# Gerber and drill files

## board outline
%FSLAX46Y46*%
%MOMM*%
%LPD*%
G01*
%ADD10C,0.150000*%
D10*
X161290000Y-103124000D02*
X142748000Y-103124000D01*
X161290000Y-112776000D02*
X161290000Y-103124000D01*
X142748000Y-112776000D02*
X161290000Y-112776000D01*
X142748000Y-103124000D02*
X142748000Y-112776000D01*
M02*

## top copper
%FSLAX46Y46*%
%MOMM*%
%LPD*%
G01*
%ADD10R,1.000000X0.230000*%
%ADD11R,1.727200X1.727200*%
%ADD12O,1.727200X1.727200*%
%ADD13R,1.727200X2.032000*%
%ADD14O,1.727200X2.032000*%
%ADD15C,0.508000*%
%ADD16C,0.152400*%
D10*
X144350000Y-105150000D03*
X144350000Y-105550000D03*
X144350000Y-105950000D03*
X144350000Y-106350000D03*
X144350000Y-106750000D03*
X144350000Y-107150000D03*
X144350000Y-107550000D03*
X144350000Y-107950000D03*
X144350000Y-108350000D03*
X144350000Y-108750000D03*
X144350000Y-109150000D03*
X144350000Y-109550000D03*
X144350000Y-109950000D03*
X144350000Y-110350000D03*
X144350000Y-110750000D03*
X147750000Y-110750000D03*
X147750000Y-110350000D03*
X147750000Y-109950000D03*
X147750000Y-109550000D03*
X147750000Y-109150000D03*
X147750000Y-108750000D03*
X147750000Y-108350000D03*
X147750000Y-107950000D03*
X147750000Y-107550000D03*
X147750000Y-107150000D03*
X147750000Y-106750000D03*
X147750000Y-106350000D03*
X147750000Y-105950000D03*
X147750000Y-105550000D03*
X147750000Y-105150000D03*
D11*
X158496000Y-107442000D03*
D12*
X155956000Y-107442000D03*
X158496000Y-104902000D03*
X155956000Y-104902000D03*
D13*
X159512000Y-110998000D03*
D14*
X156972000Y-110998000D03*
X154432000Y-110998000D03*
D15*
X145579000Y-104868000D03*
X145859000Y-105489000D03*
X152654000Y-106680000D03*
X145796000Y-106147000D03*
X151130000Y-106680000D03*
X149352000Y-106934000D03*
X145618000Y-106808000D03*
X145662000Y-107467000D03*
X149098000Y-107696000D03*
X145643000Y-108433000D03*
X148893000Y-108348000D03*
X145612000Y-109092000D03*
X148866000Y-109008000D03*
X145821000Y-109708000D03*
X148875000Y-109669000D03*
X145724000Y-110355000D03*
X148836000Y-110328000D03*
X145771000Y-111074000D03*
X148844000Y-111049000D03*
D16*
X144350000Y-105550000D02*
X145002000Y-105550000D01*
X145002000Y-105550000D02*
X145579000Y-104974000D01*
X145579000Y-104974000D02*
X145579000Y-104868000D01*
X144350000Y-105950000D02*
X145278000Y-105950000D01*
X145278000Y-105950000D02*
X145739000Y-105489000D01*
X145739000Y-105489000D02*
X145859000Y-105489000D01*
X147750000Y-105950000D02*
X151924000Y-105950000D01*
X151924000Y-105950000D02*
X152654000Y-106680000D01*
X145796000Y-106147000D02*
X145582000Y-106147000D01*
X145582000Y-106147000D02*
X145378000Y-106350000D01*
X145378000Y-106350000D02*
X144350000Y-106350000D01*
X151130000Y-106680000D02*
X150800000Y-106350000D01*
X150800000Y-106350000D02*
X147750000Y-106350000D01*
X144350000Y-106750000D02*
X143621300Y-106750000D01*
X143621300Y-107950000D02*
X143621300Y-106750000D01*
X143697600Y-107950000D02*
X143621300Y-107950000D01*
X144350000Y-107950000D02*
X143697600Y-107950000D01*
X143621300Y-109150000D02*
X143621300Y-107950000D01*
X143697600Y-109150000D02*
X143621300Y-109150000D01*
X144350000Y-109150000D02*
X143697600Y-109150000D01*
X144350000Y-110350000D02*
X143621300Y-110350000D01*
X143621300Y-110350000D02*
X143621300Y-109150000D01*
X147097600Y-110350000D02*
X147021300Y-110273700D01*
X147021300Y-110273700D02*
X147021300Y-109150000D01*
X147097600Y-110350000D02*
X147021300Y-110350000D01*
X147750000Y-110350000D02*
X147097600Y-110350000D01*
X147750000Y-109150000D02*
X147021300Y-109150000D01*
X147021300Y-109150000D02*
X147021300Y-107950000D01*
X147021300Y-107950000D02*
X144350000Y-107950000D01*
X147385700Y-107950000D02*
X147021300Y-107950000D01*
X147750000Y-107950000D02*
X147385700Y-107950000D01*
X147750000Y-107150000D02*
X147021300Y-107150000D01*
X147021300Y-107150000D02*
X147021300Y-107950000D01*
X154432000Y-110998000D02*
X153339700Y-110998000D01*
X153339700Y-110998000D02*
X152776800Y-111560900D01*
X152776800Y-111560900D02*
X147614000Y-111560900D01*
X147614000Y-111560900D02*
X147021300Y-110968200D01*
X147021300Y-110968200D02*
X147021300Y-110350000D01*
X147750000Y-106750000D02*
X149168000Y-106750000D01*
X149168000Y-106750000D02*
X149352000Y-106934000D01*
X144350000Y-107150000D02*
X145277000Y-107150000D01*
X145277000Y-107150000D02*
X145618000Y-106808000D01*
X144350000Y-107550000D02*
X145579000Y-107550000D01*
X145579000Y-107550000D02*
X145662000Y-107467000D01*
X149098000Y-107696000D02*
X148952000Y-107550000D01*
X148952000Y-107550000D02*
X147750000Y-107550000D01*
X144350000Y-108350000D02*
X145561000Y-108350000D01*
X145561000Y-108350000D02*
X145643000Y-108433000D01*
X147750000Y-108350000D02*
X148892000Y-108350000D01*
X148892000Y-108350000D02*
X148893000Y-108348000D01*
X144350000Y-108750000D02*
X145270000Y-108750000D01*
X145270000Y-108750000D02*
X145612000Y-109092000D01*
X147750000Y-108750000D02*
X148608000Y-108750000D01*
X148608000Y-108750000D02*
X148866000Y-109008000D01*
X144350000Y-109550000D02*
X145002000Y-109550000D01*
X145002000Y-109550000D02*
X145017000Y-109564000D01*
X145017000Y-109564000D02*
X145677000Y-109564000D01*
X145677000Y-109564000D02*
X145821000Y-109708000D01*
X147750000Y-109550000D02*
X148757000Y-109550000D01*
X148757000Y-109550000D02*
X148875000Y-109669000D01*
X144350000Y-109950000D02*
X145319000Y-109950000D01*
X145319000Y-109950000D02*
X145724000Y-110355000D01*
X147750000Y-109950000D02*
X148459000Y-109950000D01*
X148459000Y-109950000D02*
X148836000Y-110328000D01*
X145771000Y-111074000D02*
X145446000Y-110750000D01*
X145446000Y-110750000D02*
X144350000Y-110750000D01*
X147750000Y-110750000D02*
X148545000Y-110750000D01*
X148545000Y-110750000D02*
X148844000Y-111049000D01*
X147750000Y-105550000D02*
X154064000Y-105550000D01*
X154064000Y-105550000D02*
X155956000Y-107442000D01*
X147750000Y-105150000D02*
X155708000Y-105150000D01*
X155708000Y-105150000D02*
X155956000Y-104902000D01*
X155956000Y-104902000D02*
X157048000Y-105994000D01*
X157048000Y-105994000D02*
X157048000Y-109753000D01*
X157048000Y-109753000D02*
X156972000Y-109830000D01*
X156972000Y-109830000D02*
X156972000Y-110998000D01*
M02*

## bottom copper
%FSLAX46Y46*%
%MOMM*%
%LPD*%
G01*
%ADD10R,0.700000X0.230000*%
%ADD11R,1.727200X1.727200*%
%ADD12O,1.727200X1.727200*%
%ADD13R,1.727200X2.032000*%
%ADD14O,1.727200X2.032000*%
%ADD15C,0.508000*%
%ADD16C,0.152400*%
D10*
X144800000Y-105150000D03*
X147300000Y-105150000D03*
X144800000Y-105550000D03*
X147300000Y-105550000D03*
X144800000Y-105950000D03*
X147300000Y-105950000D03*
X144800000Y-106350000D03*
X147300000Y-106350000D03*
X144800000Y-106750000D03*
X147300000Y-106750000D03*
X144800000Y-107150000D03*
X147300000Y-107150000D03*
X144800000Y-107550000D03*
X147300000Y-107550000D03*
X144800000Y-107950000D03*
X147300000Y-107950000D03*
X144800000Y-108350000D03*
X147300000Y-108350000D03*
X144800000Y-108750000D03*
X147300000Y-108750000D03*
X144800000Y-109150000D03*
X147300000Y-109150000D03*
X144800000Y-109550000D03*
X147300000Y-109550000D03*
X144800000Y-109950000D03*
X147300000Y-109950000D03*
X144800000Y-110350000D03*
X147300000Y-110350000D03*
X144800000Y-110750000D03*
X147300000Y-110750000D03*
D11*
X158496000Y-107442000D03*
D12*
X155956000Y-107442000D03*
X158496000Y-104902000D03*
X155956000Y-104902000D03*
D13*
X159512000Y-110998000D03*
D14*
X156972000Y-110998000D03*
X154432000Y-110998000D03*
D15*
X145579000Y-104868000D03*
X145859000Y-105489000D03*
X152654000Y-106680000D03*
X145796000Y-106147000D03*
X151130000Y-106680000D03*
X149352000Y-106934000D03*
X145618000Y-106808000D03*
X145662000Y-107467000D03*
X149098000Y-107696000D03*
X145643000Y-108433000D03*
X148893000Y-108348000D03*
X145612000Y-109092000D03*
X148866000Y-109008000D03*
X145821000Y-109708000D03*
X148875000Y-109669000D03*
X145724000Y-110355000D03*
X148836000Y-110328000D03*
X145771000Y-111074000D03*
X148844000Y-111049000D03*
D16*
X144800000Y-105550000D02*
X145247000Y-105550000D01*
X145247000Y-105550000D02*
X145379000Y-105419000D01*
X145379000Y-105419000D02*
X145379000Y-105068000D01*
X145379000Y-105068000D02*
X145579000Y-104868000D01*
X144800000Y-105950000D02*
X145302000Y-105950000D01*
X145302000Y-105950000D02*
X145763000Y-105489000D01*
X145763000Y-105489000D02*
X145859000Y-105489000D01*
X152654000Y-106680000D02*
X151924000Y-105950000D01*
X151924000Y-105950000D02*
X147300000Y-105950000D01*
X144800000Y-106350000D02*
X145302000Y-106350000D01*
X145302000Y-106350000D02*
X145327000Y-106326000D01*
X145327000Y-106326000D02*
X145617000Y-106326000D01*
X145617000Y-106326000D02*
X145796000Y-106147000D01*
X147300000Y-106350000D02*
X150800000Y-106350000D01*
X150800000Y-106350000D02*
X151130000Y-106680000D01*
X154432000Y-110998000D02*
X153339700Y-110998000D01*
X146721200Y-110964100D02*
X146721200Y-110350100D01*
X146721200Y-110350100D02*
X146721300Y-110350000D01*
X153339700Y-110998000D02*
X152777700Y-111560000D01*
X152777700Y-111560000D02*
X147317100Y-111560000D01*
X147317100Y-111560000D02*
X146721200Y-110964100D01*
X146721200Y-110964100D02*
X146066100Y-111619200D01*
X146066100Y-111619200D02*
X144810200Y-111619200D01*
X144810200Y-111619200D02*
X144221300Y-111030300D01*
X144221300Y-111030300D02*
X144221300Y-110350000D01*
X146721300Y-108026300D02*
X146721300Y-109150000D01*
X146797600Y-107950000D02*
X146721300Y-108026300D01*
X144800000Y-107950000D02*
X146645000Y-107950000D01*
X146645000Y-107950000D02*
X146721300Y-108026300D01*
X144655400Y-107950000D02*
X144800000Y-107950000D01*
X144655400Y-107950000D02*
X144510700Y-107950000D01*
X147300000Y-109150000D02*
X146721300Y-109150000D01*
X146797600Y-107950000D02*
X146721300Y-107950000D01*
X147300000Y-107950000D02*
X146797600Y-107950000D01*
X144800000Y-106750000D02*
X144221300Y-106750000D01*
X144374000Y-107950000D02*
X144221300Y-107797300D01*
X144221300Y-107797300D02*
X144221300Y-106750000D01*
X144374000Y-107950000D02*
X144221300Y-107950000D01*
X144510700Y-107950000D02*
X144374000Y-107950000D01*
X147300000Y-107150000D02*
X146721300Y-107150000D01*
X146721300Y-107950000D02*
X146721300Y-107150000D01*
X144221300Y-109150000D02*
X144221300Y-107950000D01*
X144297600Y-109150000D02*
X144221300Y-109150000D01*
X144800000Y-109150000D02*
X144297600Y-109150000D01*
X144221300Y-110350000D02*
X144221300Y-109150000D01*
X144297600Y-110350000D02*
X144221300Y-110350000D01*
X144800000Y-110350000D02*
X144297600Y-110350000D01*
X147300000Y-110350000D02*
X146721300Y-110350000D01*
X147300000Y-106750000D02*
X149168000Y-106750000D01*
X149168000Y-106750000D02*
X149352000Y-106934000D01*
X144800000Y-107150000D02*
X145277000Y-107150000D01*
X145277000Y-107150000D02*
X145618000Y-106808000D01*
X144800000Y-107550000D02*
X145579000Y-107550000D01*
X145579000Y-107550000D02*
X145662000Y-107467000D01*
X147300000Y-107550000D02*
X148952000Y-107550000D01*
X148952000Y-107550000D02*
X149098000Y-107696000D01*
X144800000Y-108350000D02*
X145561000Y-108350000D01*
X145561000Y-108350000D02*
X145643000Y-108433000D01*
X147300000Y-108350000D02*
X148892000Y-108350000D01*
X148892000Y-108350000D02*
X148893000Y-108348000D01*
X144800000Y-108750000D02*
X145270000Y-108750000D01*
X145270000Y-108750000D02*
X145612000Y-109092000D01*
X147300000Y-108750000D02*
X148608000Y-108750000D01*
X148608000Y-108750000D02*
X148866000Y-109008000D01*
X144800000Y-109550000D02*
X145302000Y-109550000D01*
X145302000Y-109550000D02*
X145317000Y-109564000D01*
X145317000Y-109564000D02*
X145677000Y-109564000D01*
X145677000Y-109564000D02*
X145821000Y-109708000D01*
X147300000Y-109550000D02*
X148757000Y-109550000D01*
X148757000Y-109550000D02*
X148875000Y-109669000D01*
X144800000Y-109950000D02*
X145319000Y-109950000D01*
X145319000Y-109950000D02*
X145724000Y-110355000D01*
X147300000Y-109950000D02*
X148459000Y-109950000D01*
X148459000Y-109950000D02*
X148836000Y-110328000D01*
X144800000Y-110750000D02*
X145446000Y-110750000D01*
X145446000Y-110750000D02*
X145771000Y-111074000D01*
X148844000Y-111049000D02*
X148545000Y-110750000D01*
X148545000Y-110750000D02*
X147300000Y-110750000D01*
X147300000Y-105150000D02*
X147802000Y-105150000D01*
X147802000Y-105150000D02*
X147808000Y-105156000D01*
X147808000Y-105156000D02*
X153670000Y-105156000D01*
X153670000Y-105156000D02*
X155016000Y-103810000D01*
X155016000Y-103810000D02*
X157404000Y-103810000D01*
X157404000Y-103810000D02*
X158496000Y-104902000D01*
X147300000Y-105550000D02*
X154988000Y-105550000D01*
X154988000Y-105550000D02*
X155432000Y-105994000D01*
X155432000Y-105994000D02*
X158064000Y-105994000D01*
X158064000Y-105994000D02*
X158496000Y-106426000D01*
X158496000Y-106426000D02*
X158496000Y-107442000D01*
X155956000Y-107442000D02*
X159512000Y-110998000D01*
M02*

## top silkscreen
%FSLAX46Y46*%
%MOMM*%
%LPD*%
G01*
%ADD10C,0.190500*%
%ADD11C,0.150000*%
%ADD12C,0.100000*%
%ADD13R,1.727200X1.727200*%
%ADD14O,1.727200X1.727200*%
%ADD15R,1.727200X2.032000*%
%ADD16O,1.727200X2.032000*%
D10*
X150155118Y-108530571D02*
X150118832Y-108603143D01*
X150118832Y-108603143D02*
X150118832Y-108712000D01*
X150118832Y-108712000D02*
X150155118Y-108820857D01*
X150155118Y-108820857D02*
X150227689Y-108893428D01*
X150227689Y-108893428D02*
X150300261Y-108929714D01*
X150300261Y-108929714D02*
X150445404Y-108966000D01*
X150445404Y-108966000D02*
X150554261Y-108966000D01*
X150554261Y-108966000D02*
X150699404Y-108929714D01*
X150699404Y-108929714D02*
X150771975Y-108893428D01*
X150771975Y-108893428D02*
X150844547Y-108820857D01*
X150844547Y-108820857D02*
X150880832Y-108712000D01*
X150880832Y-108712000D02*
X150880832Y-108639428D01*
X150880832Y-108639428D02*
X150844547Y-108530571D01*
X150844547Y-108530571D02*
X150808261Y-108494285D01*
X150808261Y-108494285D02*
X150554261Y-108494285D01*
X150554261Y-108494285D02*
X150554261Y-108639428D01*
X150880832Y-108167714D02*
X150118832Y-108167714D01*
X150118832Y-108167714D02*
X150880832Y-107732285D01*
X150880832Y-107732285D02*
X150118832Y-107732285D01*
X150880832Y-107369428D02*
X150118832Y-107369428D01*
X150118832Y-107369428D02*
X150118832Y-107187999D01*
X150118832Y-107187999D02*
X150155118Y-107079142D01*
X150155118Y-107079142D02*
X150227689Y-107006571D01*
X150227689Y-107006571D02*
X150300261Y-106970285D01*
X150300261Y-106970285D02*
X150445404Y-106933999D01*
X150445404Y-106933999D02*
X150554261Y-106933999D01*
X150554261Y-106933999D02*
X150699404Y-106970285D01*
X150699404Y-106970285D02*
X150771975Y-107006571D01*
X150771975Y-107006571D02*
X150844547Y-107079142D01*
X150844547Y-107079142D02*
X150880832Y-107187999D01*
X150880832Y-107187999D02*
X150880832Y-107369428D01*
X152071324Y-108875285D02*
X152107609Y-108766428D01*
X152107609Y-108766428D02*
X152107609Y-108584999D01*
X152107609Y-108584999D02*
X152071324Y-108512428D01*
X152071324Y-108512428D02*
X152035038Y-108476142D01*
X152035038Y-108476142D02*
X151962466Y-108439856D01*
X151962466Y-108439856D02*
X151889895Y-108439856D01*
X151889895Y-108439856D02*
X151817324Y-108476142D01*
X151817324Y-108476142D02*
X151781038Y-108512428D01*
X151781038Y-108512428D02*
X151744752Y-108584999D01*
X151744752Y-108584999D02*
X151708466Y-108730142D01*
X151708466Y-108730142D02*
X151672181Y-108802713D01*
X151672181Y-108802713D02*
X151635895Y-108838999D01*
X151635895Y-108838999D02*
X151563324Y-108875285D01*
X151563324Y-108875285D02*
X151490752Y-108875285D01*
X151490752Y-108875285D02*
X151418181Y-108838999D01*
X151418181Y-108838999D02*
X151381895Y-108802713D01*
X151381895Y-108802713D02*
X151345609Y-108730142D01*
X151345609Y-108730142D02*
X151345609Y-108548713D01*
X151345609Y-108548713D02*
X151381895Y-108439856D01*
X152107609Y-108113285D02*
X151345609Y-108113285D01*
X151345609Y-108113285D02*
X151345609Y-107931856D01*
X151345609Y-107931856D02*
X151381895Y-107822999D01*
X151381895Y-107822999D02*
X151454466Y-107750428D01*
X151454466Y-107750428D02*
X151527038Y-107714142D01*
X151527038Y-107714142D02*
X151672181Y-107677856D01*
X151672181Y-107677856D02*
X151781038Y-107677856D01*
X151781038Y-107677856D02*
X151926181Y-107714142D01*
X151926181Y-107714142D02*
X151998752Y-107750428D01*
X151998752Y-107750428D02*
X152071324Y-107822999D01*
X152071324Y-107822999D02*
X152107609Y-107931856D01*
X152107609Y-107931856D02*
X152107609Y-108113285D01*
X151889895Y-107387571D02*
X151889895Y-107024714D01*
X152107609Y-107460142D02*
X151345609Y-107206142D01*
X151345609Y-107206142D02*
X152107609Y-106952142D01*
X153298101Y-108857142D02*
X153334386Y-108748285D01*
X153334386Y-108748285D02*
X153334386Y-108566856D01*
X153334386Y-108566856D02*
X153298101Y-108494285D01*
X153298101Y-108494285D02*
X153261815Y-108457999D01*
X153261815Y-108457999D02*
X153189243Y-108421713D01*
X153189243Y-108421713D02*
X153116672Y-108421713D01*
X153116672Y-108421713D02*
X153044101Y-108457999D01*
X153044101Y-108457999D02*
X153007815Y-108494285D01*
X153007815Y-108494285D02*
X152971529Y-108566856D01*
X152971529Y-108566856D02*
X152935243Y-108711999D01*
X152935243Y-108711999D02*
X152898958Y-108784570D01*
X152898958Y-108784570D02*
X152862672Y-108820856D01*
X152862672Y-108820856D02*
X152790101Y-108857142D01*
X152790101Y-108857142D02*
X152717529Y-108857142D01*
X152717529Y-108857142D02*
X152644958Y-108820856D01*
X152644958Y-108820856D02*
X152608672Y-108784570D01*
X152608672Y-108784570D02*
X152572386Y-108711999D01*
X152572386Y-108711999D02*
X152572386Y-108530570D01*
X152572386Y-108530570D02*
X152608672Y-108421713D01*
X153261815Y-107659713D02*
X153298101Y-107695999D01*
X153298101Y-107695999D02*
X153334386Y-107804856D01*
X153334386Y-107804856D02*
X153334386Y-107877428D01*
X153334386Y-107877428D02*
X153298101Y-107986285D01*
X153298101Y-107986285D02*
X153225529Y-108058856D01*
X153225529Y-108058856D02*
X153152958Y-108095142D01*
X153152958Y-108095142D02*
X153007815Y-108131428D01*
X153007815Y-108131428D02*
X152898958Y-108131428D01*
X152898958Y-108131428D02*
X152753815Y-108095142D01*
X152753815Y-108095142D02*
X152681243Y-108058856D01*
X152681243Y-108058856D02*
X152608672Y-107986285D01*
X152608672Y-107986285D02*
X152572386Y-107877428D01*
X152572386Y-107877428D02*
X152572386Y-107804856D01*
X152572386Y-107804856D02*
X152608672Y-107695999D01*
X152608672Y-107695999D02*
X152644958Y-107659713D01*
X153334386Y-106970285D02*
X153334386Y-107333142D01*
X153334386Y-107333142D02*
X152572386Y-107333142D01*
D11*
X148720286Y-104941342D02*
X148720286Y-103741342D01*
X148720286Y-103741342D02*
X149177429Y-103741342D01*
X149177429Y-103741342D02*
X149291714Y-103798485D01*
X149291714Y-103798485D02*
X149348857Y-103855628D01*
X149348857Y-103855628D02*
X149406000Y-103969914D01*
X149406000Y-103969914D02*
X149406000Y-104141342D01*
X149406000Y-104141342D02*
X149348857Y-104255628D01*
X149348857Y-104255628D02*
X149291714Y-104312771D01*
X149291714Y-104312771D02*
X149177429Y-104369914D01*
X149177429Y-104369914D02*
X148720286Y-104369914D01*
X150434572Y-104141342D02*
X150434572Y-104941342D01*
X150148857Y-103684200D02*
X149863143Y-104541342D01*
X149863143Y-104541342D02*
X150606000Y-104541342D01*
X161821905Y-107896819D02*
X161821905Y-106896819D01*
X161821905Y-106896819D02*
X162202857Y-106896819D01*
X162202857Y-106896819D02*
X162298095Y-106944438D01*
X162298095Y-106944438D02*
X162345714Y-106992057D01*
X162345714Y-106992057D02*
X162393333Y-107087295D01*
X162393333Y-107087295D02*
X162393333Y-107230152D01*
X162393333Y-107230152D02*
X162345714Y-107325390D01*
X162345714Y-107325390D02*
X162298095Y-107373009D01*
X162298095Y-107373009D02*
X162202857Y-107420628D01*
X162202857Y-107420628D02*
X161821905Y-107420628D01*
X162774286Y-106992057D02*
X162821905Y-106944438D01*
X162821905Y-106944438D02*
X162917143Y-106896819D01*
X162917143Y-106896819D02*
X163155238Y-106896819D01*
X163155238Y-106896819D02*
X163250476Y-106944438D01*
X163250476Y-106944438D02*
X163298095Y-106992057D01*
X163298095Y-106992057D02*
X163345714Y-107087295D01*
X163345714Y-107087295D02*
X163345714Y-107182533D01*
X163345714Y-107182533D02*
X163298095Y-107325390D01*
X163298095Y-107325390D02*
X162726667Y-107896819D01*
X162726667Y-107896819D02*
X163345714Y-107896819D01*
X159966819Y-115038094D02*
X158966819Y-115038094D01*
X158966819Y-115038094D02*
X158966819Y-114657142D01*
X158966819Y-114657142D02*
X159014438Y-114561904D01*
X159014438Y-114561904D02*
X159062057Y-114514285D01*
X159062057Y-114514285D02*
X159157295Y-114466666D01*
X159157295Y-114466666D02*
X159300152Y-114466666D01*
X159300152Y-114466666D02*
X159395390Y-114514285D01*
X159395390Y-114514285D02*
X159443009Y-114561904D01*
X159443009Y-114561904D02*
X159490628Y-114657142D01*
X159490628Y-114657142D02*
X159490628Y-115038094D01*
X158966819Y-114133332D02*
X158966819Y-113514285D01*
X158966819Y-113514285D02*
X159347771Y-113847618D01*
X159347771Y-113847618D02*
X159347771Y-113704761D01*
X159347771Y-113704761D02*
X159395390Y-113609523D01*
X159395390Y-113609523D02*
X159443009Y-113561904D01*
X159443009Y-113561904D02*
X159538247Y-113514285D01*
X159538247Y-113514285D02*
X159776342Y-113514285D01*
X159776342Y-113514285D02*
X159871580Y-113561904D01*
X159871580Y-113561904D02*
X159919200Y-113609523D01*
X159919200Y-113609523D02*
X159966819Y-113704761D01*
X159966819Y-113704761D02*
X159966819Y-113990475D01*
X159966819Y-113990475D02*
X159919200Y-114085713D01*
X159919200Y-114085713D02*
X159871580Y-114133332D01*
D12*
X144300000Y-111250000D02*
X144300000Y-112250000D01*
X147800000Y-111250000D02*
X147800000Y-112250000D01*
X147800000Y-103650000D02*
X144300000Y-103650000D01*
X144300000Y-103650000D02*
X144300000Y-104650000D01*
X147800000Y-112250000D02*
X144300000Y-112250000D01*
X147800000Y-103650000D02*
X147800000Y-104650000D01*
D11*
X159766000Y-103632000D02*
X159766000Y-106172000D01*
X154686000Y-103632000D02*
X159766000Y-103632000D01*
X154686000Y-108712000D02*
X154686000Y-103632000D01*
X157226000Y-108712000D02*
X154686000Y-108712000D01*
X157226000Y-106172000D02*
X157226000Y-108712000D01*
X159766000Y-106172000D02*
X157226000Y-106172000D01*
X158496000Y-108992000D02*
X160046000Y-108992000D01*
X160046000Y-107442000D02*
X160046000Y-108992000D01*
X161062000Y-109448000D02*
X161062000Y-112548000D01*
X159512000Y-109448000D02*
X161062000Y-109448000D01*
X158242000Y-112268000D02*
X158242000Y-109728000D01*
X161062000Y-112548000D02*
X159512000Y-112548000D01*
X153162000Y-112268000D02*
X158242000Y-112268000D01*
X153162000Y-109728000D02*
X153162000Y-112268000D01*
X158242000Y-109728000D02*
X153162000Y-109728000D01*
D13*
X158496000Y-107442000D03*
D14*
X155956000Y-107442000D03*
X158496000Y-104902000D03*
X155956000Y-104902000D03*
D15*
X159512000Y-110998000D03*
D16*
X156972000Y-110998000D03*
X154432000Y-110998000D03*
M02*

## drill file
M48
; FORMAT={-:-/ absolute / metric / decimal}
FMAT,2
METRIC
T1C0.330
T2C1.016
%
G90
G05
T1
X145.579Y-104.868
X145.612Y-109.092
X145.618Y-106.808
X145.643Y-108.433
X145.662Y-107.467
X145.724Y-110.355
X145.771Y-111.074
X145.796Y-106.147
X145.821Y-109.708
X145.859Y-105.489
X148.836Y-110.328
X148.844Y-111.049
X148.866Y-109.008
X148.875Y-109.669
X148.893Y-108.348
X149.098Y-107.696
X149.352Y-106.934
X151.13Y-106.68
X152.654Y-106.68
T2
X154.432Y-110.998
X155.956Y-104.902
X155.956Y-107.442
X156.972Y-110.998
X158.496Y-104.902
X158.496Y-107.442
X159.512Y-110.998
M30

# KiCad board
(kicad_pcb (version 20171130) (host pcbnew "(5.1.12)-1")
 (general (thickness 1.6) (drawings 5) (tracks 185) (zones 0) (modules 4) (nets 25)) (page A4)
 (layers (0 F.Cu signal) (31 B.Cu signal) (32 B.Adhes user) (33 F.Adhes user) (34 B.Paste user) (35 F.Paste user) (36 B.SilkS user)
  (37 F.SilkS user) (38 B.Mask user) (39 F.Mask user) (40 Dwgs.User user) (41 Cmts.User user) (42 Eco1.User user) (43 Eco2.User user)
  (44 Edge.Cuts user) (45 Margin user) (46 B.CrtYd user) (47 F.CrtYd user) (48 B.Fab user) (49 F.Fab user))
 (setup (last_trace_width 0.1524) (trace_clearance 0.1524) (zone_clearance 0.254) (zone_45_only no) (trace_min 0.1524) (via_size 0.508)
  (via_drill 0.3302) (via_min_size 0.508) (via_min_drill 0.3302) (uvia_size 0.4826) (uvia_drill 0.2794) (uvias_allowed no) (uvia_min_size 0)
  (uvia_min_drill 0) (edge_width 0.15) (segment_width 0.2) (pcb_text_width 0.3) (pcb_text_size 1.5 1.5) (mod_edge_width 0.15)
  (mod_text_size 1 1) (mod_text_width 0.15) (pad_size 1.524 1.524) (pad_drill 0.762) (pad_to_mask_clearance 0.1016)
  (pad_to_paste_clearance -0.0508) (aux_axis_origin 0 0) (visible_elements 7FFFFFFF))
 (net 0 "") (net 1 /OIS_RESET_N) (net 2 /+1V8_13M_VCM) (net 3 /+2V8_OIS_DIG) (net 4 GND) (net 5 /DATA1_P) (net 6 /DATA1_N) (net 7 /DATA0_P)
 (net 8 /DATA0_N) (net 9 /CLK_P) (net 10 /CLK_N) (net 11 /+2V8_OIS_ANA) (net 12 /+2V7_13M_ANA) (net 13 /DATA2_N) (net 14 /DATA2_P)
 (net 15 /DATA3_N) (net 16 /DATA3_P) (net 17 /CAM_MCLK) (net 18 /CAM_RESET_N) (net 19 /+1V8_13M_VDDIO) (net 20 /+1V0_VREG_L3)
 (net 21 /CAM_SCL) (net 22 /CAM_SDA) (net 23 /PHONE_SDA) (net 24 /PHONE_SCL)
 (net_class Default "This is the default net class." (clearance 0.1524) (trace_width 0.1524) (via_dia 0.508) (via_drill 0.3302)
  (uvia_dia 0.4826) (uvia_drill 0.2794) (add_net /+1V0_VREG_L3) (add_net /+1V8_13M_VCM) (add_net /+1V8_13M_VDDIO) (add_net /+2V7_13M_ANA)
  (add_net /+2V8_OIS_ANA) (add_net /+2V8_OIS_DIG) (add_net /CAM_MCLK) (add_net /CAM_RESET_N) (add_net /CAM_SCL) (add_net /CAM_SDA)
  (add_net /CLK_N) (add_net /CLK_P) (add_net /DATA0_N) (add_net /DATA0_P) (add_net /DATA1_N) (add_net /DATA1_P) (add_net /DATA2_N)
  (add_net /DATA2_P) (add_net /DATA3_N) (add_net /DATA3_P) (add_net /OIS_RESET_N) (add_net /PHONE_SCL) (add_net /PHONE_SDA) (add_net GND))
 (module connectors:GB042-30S (layer F.Cu) (at 146.05 107.95 270)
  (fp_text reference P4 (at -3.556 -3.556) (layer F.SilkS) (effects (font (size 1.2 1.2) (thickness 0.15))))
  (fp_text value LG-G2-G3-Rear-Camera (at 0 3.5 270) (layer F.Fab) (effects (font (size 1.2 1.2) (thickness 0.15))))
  (fp_line (start 3.3 1.75) (end 4.3 1.75) (layer F.SilkS) (width 0.1))
  (fp_line (start 3.3 -1.75) (end 4.3 -1.75) (layer F.SilkS) (width 0.1))
  (fp_line (start -4.3 -1.75) (end -4.3 1.75) (layer F.SilkS) (width 0.1))
  (fp_line (start -4.3 1.75) (end -3.3 1.75) (layer F.SilkS) (width 0.1))
  (fp_line (start 4.3 -1.75) (end 4.3 1.75) (layer F.SilkS) (width 0.1))
  (fp_line (start -4.3 -1.75) (end -3.3 -1.75) (layer F.SilkS) (width 0.1))
  (pad 1 smd rect (at -2.8 1.7 90) (size 0.23 1) (layers F.Cu F.Paste F.Mask))
  (pad 2 smd rect (at -2.4 1.7 90) (size 0.23 1) (layers F.Cu F.Paste F.Mask) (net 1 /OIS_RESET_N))
  (pad 3 smd rect (at -2 1.7 90) (size 0.23 1) (layers F.Cu F.Paste F.Mask) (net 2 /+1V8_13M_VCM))
  (pad 4 smd rect (at -1.6 1.7 90) (size 0.23 1) (layers F.Cu F.Paste F.Mask) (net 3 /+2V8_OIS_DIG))
  (pad 5 smd rect (at -1.2 1.7 90) (size 0.23 1) (layers F.Cu F.Paste F.Mask) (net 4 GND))
  (pad 6 smd rect (at -0.8 1.7 90) (size 0.23 1) (layers F.Cu F.Paste F.Mask) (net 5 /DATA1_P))
  (pad 7 smd rect (at -0.4 1.7 90) (size 0.23 1) (layers F.Cu F.Paste F.Mask) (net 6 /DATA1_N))
  (pad 8 smd rect (at 0 1.7 90) (size 0.23 1) (layers F.Cu F.Paste F.Mask) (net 4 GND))
  (pad 9 smd rect (at 0.4 1.7 90) (size 0.23 1) (layers F.Cu F.Paste F.Mask) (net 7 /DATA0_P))
  (pad 10 smd rect (at 0.8 1.7 90) (size 0.23 1) (layers F.Cu F.Paste F.Mask) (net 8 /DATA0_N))
  (pad 11 smd rect (at 1.2 1.7 90) (size 0.23 1) (layers F.Cu F.Paste F.Mask) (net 4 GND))
  (pad 12 smd rect (at 1.6 1.7 90) (size 0.23 1) (layers F.Cu F.Paste F.Mask) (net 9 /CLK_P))
  (pad 13 smd rect (at 2 1.7 90) (size 0.23 1) (layers F.Cu F.Paste F.Mask) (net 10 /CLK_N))
  (pad 14 smd rect (at 2.4 1.7 90) (size 0.23 1) (layers F.Cu F.Paste F.Mask) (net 4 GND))
  (pad 15 smd rect (at 2.8 1.7 90) (size 0.23 1) (layers F.Cu F.Paste F.Mask) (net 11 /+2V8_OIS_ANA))
  (pad 16 smd rect (at 2.8 -1.7 270) (size 0.23 1) (layers F.Cu F.Paste F.Mask) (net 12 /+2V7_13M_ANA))
  (pad 17 smd rect (at 2.4 -1.7 270) (size 0.23 1) (layers F.Cu F.Paste F.Mask) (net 4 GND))
  (pad 18 smd rect (at 2 -1.7 270) (size 0.23 1) (layers F.Cu F.Paste F.Mask) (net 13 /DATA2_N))
  (pad 19 smd rect (at 1.6 -1.7 270) (size 0.23 1) (layers F.Cu F.Paste F.Mask) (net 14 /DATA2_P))
  (pad 20 smd rect (at 1.2 -1.7 270) (size 0.23 1) (layers F.Cu F.Paste F.Mask) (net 4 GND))
  (pad 21 smd rect (at 0.8 -1.7 270) (size 0.23 1) (layers F.Cu F.Paste F.Mask) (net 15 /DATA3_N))
  (pad 22 smd rect (at 0.4 -1.7 270) (size 0.23 1) (layers F.Cu F.Paste F.Mask) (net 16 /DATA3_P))
  (pad 23 smd rect (at 0 -1.7 270) (size 0.23 1) (layers F.Cu F.Paste F.Mask) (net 4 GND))
  (pad 24 smd rect (at -0.4 -1.7 270) (size 0.23 1) (layers F.Cu F.Paste F.Mask) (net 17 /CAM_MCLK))
  (pad 25 smd rect (at -0.8 -1.7 270) (size 0.23 1) (layers F.Cu F.Paste F.Mask) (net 4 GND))
  (pad 26 smd rect (at -1.2 -1.7 270) (size 0.23 1) (layers F.Cu F.Paste F.Mask) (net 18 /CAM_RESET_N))
  (pad 27 smd rect (at -1.6 -1.7 270) (size 0.23 1) (layers F.Cu F.Paste F.Mask) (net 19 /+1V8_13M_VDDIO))
  (pad 28 smd rect (at -2 -1.7 270) (size 0.23 1) (layers F.Cu F.Paste F.Mask) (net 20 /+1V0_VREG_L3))
  (pad 29 smd rect (at -2.4 -1.7 270) (size 0.23 1) (layers F.Cu F.Paste F.Mask) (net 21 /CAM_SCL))
  (pad 30 smd rect (at -2.8 -1.7 270) (size 0.23 1) (layers F.Cu F.Paste F.Mask) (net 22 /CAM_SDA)))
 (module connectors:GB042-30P (layer B.Cu) (at 146.05 107.95 270)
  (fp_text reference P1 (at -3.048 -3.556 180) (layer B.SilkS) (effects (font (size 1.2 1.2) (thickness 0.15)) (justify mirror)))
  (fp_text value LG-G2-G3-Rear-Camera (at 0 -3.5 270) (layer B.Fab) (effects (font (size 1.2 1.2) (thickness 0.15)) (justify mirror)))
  (pad 1 smd rect (at -2.8 1.25 270) (size 0.23 0.7) (layers B.Cu B.Paste B.Mask))
  (pad 30 smd rect (at -2.8 -1.25 270) (size 0.23 0.7) (layers B.Cu B.Paste B.Mask) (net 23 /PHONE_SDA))
  (pad 2 smd rect (at -2.4 1.25 270) (size 0.23 0.7) (layers B.Cu B.Paste B.Mask) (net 1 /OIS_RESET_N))
  (pad 29 smd rect (at -2.4 -1.25 270) (size 0.23 0.7) (layers B.Cu B.Paste B.Mask) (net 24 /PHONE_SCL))
  (pad 3 smd rect (at -2 1.25 270) (size 0.23 0.7) (layers B.Cu B.Paste B.Mask) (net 2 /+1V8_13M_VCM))
  (pad 28 smd rect (at -2 -1.25 270) (size 0.23 0.7) (layers B.Cu B.Paste B.Mask) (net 20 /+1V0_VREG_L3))
  (pad 4 smd rect (at -1.6 1.25 270) (size 0.23 0.7) (layers B.Cu B.Paste B.Mask) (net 3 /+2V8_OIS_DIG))
  (pad 27 smd rect (at -1.6 -1.25 270) (size 0.23 0.7) (layers B.Cu B.Paste B.Mask) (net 19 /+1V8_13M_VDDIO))
  (pad 5 smd rect (at -1.2 1.25 270) (size 0.23 0.7) (layers B.Cu B.Paste B.Mask) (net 4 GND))
  (pad 26 smd rect (at -1.2 -1.25 270) (size 0.23 0.7) (layers B.Cu B.Paste B.Mask) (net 18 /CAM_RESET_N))
  (pad 6 smd rect (at -0.8 1.25 270) (size 0.23 0.7) (layers B.Cu B.Paste B.Mask) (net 5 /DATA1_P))
  (pad 25 smd rect (at -0.8 -1.25 270) (size 0.23 0.7) (layers B.Cu B.Paste B.Mask) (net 4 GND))
  (pad 7 smd rect (at -0.4 1.25 270) (size 0.23 0.7) (layers B.Cu B.Paste B.Mask) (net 6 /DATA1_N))
  (pad 24 smd rect (at -0.4 -1.25 270) (size 0.23 0.7) (layers B.Cu B.Paste B.Mask) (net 17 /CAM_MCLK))
  (pad 8 smd rect (at 0 1.25 270) (size 0.23 0.7) (layers B.Cu B.Paste B.Mask) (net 4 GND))
  (pad 23 smd rect (at 0 -1.25 270) (size 0.23 0.7) (layers B.Cu B.Paste B.Mask) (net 4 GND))
  (pad 9 smd rect (at 0.4 1.25 270) (size 0.23 0.7) (layers B.Cu B.Paste B.Mask) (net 7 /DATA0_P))
  (pad 22 smd rect (at 0.4 -1.25 270) (size 0.23 0.7) (layers B.Cu B.Paste B.Mask) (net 16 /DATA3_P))
  (pad 10 smd rect (at 0.8 1.25 270) (size 0.23 0.7) (layers B.Cu B.Paste B.Mask) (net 8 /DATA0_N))
  (pad 21 smd rect (at 0.8 -1.25 270) (size 0.23 0.7) (layers B.Cu B.Paste B.Mask) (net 15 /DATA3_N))
  (pad 11 smd rect (at 1.2 1.25 270) (size 0.23 0.7) (layers B.Cu B.Paste B.Mask) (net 4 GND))
  (pad 20 smd rect (at 1.2 -1.25 270) (size 0.23 0.7) (layers B.Cu B.Paste B.Mask) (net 4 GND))
  (pad 12 smd rect (at 1.6 1.25 270) (size 0.23 0.7) (layers B.Cu B.Paste B.Mask) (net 9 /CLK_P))
  (pad 19 smd rect (at 1.6 -1.25 270) (size 0.23 0.7) (layers B.Cu B.Paste B.Mask) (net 14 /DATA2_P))
  (pad 13 smd rect (at 2 1.25 270) (size 0.23 0.7) (layers B.Cu B.Paste B.Mask) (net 10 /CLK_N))
  (pad 18 smd rect (at 2 -1.25 270) (size 0.23 0.7) (layers B.Cu B.Paste B.Mask) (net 13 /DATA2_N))
  (pad 14 smd rect (at 2.4 1.25 270) (size 0.23 0.7) (layers B.Cu B.Paste B.Mask) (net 4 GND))
  (pad 17 smd rect (at 2.4 -1.25 270) (size 0.23 0.7) (layers B.Cu B.Paste B.Mask) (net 4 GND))
  (pad 15 smd rect (at 2.8 1.25 270) (size 0.23 0.7) (layers B.Cu B.Paste B.Mask) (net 11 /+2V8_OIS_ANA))
  (pad 16 smd rect (at 2.8 -1.25 270) (size 0.23 0.7) (layers B.Cu B.Paste B.Mask) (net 12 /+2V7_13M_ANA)))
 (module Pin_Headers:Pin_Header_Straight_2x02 (layer F.Cu) (at 158.496 107.442 180)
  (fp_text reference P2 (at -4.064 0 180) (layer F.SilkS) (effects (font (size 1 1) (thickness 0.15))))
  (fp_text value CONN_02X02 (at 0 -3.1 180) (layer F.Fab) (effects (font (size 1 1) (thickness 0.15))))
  (fp_line (start -1.27 3.81) (end -1.27 1.27) (layer F.SilkS) (width 0.15))
  (fp_line (start 3.81 3.81) (end -1.27 3.81) (layer F.SilkS) (width 0.15))
  (fp_line (start 3.81 -1.27) (end 3.81 3.81) (layer F.SilkS) (width 0.15))
  (fp_line (start 1.27 -1.27) (end 3.81 -1.27) (layer F.SilkS) (width 0.15))
  (fp_line (start 1.27 1.27) (end 1.27 -1.27) (layer F.SilkS) (width 0.15))
  (fp_line (start -1.27 1.27) (end 1.27 1.27) (layer F.SilkS) (width 0.15))
  (fp_line (start 0 -1.55) (end -1.55 -1.55) (layer F.SilkS) (width 0.15))
  (fp_line (start -1.55 0) (end -1.55 -1.55) (layer F.SilkS) (width 0.15))
  (pad 1 thru_hole rect (at 0 0 180) (size 1.7272 1.7272) (drill 1.016) (layers *.Cu *.Mask F.SilkS) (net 24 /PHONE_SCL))
  (pad 2 thru_hole oval (at 2.54 0 180) (size 1.7272 1.7272) (drill 1.016) (layers *.Cu *.Mask F.SilkS) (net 21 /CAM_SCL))
  (pad 3 thru_hole oval (at 0 2.54 180) (size 1.7272 1.7272) (drill 1.016) (layers *.Cu *.Mask F.SilkS) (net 23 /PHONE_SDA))
  (pad 4 thru_hole oval (at 2.54 2.54 180) (size 1.7272 1.7272) (drill 1.016) (layers *.Cu *.Mask F.SilkS) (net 22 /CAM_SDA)))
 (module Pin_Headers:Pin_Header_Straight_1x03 (layer F.Cu) (at 159.512 110.998 270)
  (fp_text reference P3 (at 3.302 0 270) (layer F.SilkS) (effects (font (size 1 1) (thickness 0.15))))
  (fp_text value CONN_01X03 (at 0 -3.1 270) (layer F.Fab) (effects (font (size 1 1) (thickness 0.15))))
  (fp_line (start -1.55 -1.55) (end 1.55 -1.55) (layer F.SilkS) (width 0.15))
  (fp_line (start -1.55 0) (end -1.55 -1.55) (layer F.SilkS) (width 0.15))
  (fp_line (start 1.27 1.27) (end -1.27 1.27) (layer F.SilkS) (width 0.15))
  (fp_line (start 1.55 -1.55) (end 1.55 0) (layer F.SilkS) (width 0.15))
  (fp_line (start 1.27 6.35) (end 1.27 1.27) (layer F.SilkS) (width 0.15))
  (fp_line (start -1.27 6.35) (end 1.27 6.35) (layer F.SilkS) (width 0.15))
  (fp_line (start -1.27 1.27) (end -1.27 6.35) (layer F.SilkS) (width 0.15))
  (pad 1 thru_hole rect (at 0 0 270) (size 2.032 1.7272) (drill 1.016) (layers *.Cu *.Mask F.SilkS) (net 21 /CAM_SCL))
  (pad 2 thru_hole oval (at 0 2.54 270) (size 2.032 1.7272) (drill 1.016) (layers *.Cu *.Mask F.SilkS) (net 22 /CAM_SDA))
  (pad 3 thru_hole oval (at 0 5.08 270) (size 2.032 1.7272) (drill 1.016) (layers *.Cu *.Mask F.SilkS) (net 4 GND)))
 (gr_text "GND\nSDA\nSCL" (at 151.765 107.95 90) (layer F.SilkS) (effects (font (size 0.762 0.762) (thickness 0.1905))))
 (gr_line (start 161.29 103.124) (end 142.748 103.124) (layer Edge.Cuts) (width 0.15))
 (gr_line (start 161.29 112.776) (end 161.29 103.124) (layer Edge.Cuts) (width 0.15))
 (gr_line (start 142.748 112.776) (end 161.29 112.776) (layer Edge.Cuts) (width 0.15))
 (gr_line (start 142.748 103.124) (end 142.748 112.776) (layer Edge.Cuts) (width 0.15))
 (segment (start 144.35 105.55) (end 145.002 105.55) (width 0.1524) (layer F.Cu) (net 1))
 (segment (start 145.002 105.55) (end 145.579 104.974) (width 0.1524) (layer F.Cu) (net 1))
 (segment (start 145.579 104.974) (end 145.579 104.868) (width 0.1524) (layer F.Cu) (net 1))
 (segment (start 144.8 105.55) (end 145.247 105.55) (width 0.1524) (layer B.Cu) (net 1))
 (segment (start 145.247 105.55) (end 145.379 105.419) (width 0.1524) (layer B.Cu) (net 1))
 (segment (start 145.379 105.419) (end 145.379 105.068) (width 0.1524) (layer B.Cu) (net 1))
 (segment (start 145.379 105.068) (end 145.579 104.868) (width 0.1524) (layer B.Cu) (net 1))
 (via (at 145.579 104.868) (size 0.508) (layers F.Cu B.Cu) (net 1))
 (segment (start 144.35 105.95) (end 145.278 105.95) (width 0.1524) (layer F.Cu) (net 2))
 (segment (start 145.278 105.95) (end 145.739 105.489) (width 0.1524) (layer F.Cu) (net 2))
 (segment (start 145.739 105.489) (end 145.859 105.489) (width 0.1524) (layer F.Cu) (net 2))
 (segment (start 144.8 105.95) (end 145.302 105.95) (width 0.1524) (layer B.Cu) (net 2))
 (segment (start 145.302 105.95) (end 145.763 105.489) (width 0.1524) (layer B.Cu) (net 2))
 (segment (start 145.763 105.489) (end 145.859 105.489) (width 0.1524) (layer B.Cu) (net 2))
 (via (at 145.859 105.489) (size 0.508) (layers F.Cu B.Cu) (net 2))
 (segment (start 147.75 105.95) (end 151.924 105.95) (width 0.1524) (layer F.Cu) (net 20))
 (segment (start 151.924 105.95) (end 152.654 106.68) (width 0.1524) (layer F.Cu) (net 20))
 (segment (start 152.654 106.68) (end 151.924 105.95) (width 0.1524) (layer B.Cu) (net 20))
 (segment (start 151.924 105.95) (end 147.3 105.95) (width 0.1524) (layer B.Cu) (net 20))
 (via (at 152.654 106.68) (size 0.508) (layers F.Cu B.Cu) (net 20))
 (segment (start 145.796 106.147) (end 145.582 106.147) (width 0.1524) (layer F.Cu) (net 3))
 (segment (start 145.582 106.147) (end 145.378 106.35) (width 0.1524) (layer F.Cu) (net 3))
 (segment (start 145.378 106.35) (end 144.35 106.35) (width 0.1524) (layer F.Cu) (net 3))
 (segment (start 144.8 106.35) (end 145.302 106.35) (width 0.1524) (layer B.Cu) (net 3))
 (segment (start 145.302 106.35) (end 145.327 106.326) (width 0.1524) (layer B.Cu) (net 3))
 (segment (start 145.327 106.326) (end 145.617 106.326) (width 0.1524) (layer B.Cu) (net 3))
 (segment (start 145.617 106.326) (end 145.796 106.147) (width 0.1524) (layer B.Cu) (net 3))
 (via (at 145.796 106.147) (size 0.508) (layers F.Cu B.Cu) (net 3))
 (segment (start 147.3 106.35) (end 150.8 106.35) (width 0.1524) (layer B.Cu) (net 19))
 (segment (start 150.8 106.35) (end 151.13 106.68) (width 0.1524) (layer B.Cu) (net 19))
 (segment (start 151.13 106.68) (end 150.8 106.35) (width 0.1524) (layer F.Cu) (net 19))
 (segment (start 150.8 106.35) (end 147.75 106.35) (width 0.1524) (layer F.Cu) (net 19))
 (via (at 151.13 106.68) (size 0.508) (layers F.Cu B.Cu) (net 19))
 (segment (start 154.432 110.998) (end 153.3397 110.998) (width 0.1524) (layer B.Cu) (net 4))
 (segment (start 146.7212 110.9641) (end 146.7212 110.3501) (width 0.1524) (layer B.Cu) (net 4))
 (segment (start 146.7212 110.3501) (end 146.7213 110.35) (width 0.1524) (layer B.Cu) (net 4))
 (segment (start 153.3397 110.998) (end 152.7777 111.56) (width 0.1524) (layer B.Cu) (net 4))
 (segment (start 152.7777 111.56) (end 147.3171 111.56) (width 0.1524) (layer B.Cu) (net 4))
 (segment (start 147.3171 111.56) (end 146.7212 110.9641) (width 0.1524) (layer B.Cu) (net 4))
 (segment (start 146.7212 110.9641) (end 146.0661 111.6192) (width 0.1524) (layer B.Cu) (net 4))
 (segment (start 146.0661 111.6192) (end 144.8102 111.6192) (width 0.1524) (layer B.Cu) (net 4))
 (segment (start 144.8102 111.6192) (end 144.2213 111.0303) (width 0.1524) (layer B.Cu) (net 4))
 (segment (start 144.2213 111.0303) (end 144.2213 110.35) (width 0.1524) (layer B.Cu) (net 4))
 (segment (start 144.35 106.75) (end 143.6213 106.75) (width 0.1524) (layer F.Cu) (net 4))
 (segment (start 143.6213 107.95) (end 143.6213 106.75) (width 0.1524) (layer F.Cu) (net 4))
 (segment (start 143.6976 107.95) (end 143.6213 107.95) (width 0.1524) (layer F.Cu) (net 4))
 (segment (start 144.35 107.95) (end 143.6976 107.95) (width 0.1524) (layer F.Cu) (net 4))
 (segment (start 143.6213 109.15) (end 143.6213 107.95) (width 0.1524) (layer F.Cu) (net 4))
 (segment (start 143.6976 109.15) (end 143.6213 109.15) (width 0.1524) (layer F.Cu) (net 4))
 (segment (start 144.35 109.15) (end 143.6976 109.15) (width 0.1524) (layer F.Cu) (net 4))
 (segment (start 144.35 110.35) (end 143.6213 110.35) (width 0.1524) (layer F.Cu) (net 4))
 (segment (start 143.6213 110.35) (end 143.6213 109.15) (width 0.1524) (layer F.Cu) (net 4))
 (segment (start 147.0976 110.35) (end 147.0213 110.2737) (width 0.1524) (layer F.Cu) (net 4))
 (segment (start 147.0213 110.2737) (end 147.0213 109.15) (width 0.1524) (layer F.Cu) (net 4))
 (segment (start 147.0976 110.35) (end 147.0213 110.35) (width 0.1524) (layer F.Cu) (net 4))
 (segment (start 147.75 110.35) (end 147.0976 110.35) (width 0.1524) (layer F.Cu) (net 4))
 (segment (start 147.75 109.15) (end 147.0213 109.15) (width 0.1524) (layer F.Cu) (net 4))
 (segment (start 147.0213 109.15) (end 147.0213 107.95) (width 0.1524) (layer F.Cu) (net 4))
 (segment (start 147.0213 107.95) (end 144.35 107.95) (width 0.1524) (layer F.Cu) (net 4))
 (segment (start 147.3857 107.95) (end 147.0213 107.95) (width 0.1524) (layer F.Cu) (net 4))
 (segment (start 147.75 107.95) (end 147.3857 107.95) (width 0.1524) (layer F.Cu) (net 4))
 (segment (start 147.75 107.15) (end 147.0213 107.15) (width 0.1524) (layer F.Cu) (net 4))
 (segment (start 147.0213 107.15) (end 147.0213 107.95) (width 0.1524) (layer F.Cu) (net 4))
 (segment (start 146.7213 108.0263) (end 146.7213 109.15) (width 0.1524) (layer B.Cu) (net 4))
 (segment (start 146.7976 107.95) (end 146.7213 108.0263) (width 0.1524) (layer B.Cu) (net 4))
 (segment (start 144.8 107.95) (end 146.645 107.95) (width 0.1524) (layer B.Cu) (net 4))
 (segment (start 146.645 107.95) (end 146.7213 108.0263) (width 0.1524) (layer B.Cu) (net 4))
 (segment (start 144.6554 107.95) (end 144.8 107.95) (width 0.1524) (layer B.Cu) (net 4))
 (segment (start 144.6554 107.95) (end 144.5107 107.95) (width 0.1524) (layer B.Cu) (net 4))
 (segment (start 147.3 109.15) (end 146.7213 109.15) (width 0.1524) (layer B.Cu) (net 4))
 (segment (start 146.7976 107.95) (end 146.7213 107.95) (width 0.1524) (layer B.Cu) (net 4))
 (segment (start 147.3 107.95) (end 146.7976 107.95) (width 0.1524) (layer B.Cu) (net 4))
 (segment (start 144.8 106.75) (end 144.2213 106.75) (width 0.1524) (layer B.Cu) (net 4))
 (segment (start 144.374 107.95) (end 144.2213 107.7973) (width 0.1524) (layer B.Cu) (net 4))
 (segment (start 144.2213 107.7973) (end 144.2213 106.75) (width 0.1524) (layer B.Cu) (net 4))
 (segment (start 144.374 107.95) (end 144.2213 107.95) (width 0.1524) (layer B.Cu) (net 4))
 (segment (start 144.5107 107.95) (end 144.374 107.95) (width 0.1524) (layer B.Cu) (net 4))
 (segment (start 147.3 107.15) (end 146.7213 107.15) (width 0.1524) (layer B.Cu) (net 4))
 (segment (start 146.7213 107.95) (end 146.7213 107.15) (width 0.1524) (layer B.Cu) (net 4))
 (segment (start 144.2213 109.15) (end 144.2213 107.95) (width 0.1524) (layer B.Cu) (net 4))
 (segment (start 144.2976 109.15) (end 144.2213 109.15) (width 0.1524) (layer B.Cu) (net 4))
 (segment (start 144.8 109.15) (end 144.2976 109.15) (width 0.1524) (layer B.Cu) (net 4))
 (segment (start 144.2213 110.35) (end 144.2213 109.15) (width 0.1524) (layer B.Cu) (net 4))
 (segment (start 144.2976 110.35) (end 144.2213 110.35) (width 0.1524) (layer B.Cu) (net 4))
 (segment (start 144.8 110.35) (end 144.2976 110.35) (width 0.1524) (layer B.Cu) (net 4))
 (segment (start 147.3 110.35) (end 146.7213 110.35) (width 0.1524) (layer B.Cu) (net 4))
 (segment (start 154.432 110.998) (end 153.3397 110.998) (width 0.1524) (layer F.Cu) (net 4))
 (segment (start 153.3397 110.998) (end 152.7768 111.5609) (width 0.1524) (layer F.Cu) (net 4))
 (segment (start 152.7768 111.5609) (end 147.614 111.5609) (width 0.1524) (layer F.Cu) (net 4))
 (segment (start 147.614 111.5609) (end 147.0213 110.9682) (width 0.1524) (layer F.Cu) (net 4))
 (segment (start 147.0213 110.9682) (end 147.0213 110.35) (width 0.1524) (layer F.Cu) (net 4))
 (segment (start 147.3 106.75) (end 149.168 106.75) (width 0.1524) (layer B.Cu) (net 18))
 (segment (start 149.168 106.75) (end 149.352 106.934) (width 0.1524) (layer B.Cu) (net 18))
 (segment (start 147.75 106.75) (end 149.168 106.75) (width 0.1524) (layer F.Cu) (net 18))
 (segment (start 149.168 106.75) (end 149.352 106.934) (width 0.1524) (layer F.Cu) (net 18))
 (via (at 149.352 106.934) (size 0.508) (layers F.Cu B.Cu) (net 18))
 (segment (start 144.35 107.15) (end 145.277 107.15) (width 0.1524) (layer F.Cu) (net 5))
 (segment (start 145.277 107.15) (end 145.618 106.808) (width 0.1524) (layer F.Cu) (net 5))
 (segment (start 144.8 107.15) (end 145.277 107.15) (width 0.1524) (layer B.Cu) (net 5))
 (segment (start 145.277 107.15) (end 145.618 106.808) (width 0.1524) (layer B.Cu) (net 5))
 (via (at 145.618 106.808) (size 0.508) (layers F.Cu B.Cu) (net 5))
 (segment (start 144.35 107.55) (end 145.579 107.55) (width 0.1524) (layer F.Cu) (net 6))
 (segment (start 145.579 107.55) (end 145.662 107.467) (width 0.1524) (layer F.Cu) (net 6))
 (segment (start 144.8 107.55) (end 145.579 107.55) (width 0.1524) (layer B.Cu) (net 6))
 (segment (start 145.579 107.55) (end 145.662 107.467) (width 0.1524) (layer B.Cu) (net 6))
 (via (at 145.662 107.467) (size 0.508) (layers F.Cu B.Cu) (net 6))
 (segment (start 147.3 107.55) (end 148.952 107.55) (width 0.1524) (layer B.Cu) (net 17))
 (segment (start 148.952 107.55) (end 149.098 107.696) (width 0.1524) (layer B.Cu) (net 17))
 (segment (start 149.098 107.696) (end 148.952 107.55) (width 0.1524) (layer F.Cu) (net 17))
 (segment (start 148.952 107.55) (end 147.75 107.55) (width 0.1524) (layer F.Cu) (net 17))
 (via (at 149.098 107.696) (size 0.508) (layers F.Cu B.Cu) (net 17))
 (segment (start 144.35 108.35) (end 145.561 108.35) (width 0.1524) (layer F.Cu) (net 7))
 (segment (start 145.561 108.35) (end 145.643 108.433) (width 0.1524) (layer F.Cu) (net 7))
 (segment (start 144.8 108.35) (end 145.561 108.35) (width 0.1524) (layer B.Cu) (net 7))
 (segment (start 145.561 108.35) (end 145.643 108.433) (width 0.1524) (layer B.Cu) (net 7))
 (via (at 145.643 108.433) (size 0.508) (layers F.Cu B.Cu) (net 7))
 (segment (start 147.75 108.35) (end 148.892 108.35) (width 0.1524) (layer F.Cu) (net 16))
 (segment (start 148.892 108.35) (end 148.893 108.348) (width 0.1524) (layer F.Cu) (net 16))
 (segment (start 147.3 108.35) (end 148.892 108.35) (width 0.1524) (layer B.Cu) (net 16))
 (segment (start 148.892 108.35) (end 148.893 108.348) (width 0.1524) (layer B.Cu) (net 16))
 (via (at 148.893 108.348) (size 0.508) (layers F.Cu B.Cu) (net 16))
 (segment (start 144.35 108.75) (end 145.27 108.75) (width 0.1524) (layer F.Cu) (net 8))
 (segment (start 145.27 108.75) (end 145.612 109.092) (width 0.1524) (layer F.Cu) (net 8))
 (segment (start 144.8 108.75) (end 145.27 108.75) (width 0.1524) (layer B.Cu) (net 8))
 (segment (start 145.27 108.75) (end 145.612 109.092) (width 0.1524) (layer B.Cu) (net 8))
 (via (at 145.612 109.092) (size 0.508) (layers F.Cu B.Cu) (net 8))
 (segment (start 147.3 108.75) (end 148.608 108.75) (width 0.1524) (layer B.Cu) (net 15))
 (segment (start 148.608 108.75) (end 148.866 109.008) (width 0.1524) (layer B.Cu) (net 15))
 (segment (start 147.75 108.75) (end 148.608 108.75) (width 0.1524) (layer F.Cu) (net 15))
 (segment (start 148.608 108.75) (end 148.866 109.008) (width 0.1524) (layer F.Cu) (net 15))
 (via (at 148.866 109.008) (size 0.508) (layers F.Cu B.Cu) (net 15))
 (segment (start 144.35 109.55) (end 145.002 109.55) (width 0.1524) (layer F.Cu) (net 9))
 (segment (start 145.002 109.55) (end 145.017 109.564) (width 0.1524) (layer F.Cu) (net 9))
 (segment (start 145.017 109.564) (end 145.677 109.564) (width 0.1524) (layer F.Cu) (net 9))
 (segment (start 145.677 109.564) (end 145.821 109.708) (width 0.1524) (layer F.Cu) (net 9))
 (segment (start 144.8 109.55) (end 145.302 109.55) (width 0.1524) (layer B.Cu) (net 9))
 (segment (start 145.302 109.55) (end 145.317 109.564) (width 0.1524) (layer B.Cu) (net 9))
 (segment (start 145.317 109.564) (end 145.677 109.564) (width 0.1524) (layer B.Cu) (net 9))
 (segment (start 145.677 109.564) (end 145.821 109.708) (width 0.1524) (layer B.Cu) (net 9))
 (via (at 145.821 109.708) (size 0.508) (layers F.Cu B.Cu) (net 9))
 (segment (start 147.3 109.55) (end 148.757 109.55) (width 0.1524) (layer B.Cu) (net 14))
 (segment (start 148.757 109.55) (end 148.875 109.669) (width 0.1524) (layer B.Cu) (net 14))
 (segment (start 147.75 109.55) (end 148.757 109.55) (width 0.1524) (layer F.Cu) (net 14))
 (segment (start 148.757 109.55) (end 148.875 109.669) (width 0.1524) (layer F.Cu) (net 14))
 (via (at 148.875 109.669) (size 0.508) (layers F.Cu B.Cu) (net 14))
 (segment (start 144.8 109.95) (end 145.319 109.95) (width 0.1524) (layer B.Cu) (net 10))
 (segment (start 145.319 109.95) (end 145.724 110.355) (width 0.1524) (layer B.Cu) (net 10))
 (segment (start 144.35 109.95) (end 145.319 109.95) (width 0.1524) (layer F.Cu) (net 10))
 (segment (start 145.319 109.95) (end 145.724 110.355) (width 0.1524) (layer F.Cu) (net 10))
 (via (at 145.724 110.355) (size 0.508) (layers F.Cu B.Cu) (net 10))
 (segment (start 147.3 109.95) (end 148.459 109.95) (width 0.1524) (layer B.Cu) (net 13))
 (segment (start 148.459 109.95) (end 148.836 110.328) (width 0.1524) (layer B.Cu) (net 13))
 (segment (start 147.75 109.95) (end 148.459 109.95) (width 0.1524) (layer F.Cu) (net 13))
 (segment (start 148.459 109.95) (end 148.836 110.328) (width 0.1524) (layer F.Cu) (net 13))
 (via (at 148.836 110.328) (size 0.508) (layers F.Cu B.Cu) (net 13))
 (segment (start 144.8 110.75) (end 145.446 110.75) (width 0.1524) (layer B.Cu) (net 11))
 (segment (start 145.446 110.75) (end 145.771 111.074) (width 0.1524) (layer B.Cu) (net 11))
 (segment (start 145.771 111.074) (end 145.446 110.75) (width 0.1524) (layer F.Cu) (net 11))
 (segment (start 145.446 110.75) (end 144.35 110.75) (width 0.1524) (layer F.Cu) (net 11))
 (via (at 145.771 111.074) (size 0.508) (layers F.Cu B.Cu) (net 11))
 (segment (start 147.75 110.75) (end 148.545 110.75) (width 0.1524) (layer F.Cu) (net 12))
 (segment (start 148.545 110.75) (end 148.844 111.049) (width 0.1524) (layer F.Cu) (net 12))
 (segment (start 148.844 111.049) (end 148.545 110.75) (width 0.1524) (layer B.Cu) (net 12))
 (segment (start 148.545 110.75) (end 147.3 110.75) (width 0.1524) (layer B.Cu) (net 12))
 (via (at 148.844 111.049) (size 0.508) (layers F.Cu B.Cu) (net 12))
 (segment (start 147.3 105.15) (end 147.802 105.15) (width 0.1524) (layer B.Cu) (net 23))
 (segment (start 147.802 105.15) (end 147.808 105.156) (width 0.1524) (layer B.Cu) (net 23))
 (segment (start 147.808 105.156) (end 153.67 105.156) (width 0.1524) (layer B.Cu) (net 23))
 (segment (start 153.67 105.156) (end 155.016 103.81) (width 0.1524) (layer B.Cu) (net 23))
 (segment (start 155.016 103.81) (end 157.404 103.81) (width 0.1524) (layer B.Cu) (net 23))
 (segment (start 157.404 103.81) (end 158.496 104.902) (width 0.1524) (layer B.Cu) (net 23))
 (segment (start 147.3 105.55) (end 154.988 105.55) (width 0.1524) (layer B.Cu) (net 24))
 (segment (start 154.988 105.55) (end 155.432 105.994) (width 0.1524) (layer B.Cu) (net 24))
 (segment (start 155.432 105.994) (end 158.064 105.994) (width 0.1524) (layer B.Cu) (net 24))
 (segment (start 158.064 105.994) (end 158.496 106.426) (width 0.1524) (layer B.Cu) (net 24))
 (segment (start 158.496 106.426) (end 158.496 107.442) (width 0.1524) (layer B.Cu) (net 24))
 (segment (start 147.75 105.55) (end 154.064 105.55) (width 0.1524) (layer F.Cu) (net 21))
 (segment (start 154.064 105.55) (end 155.956 107.442) (width 0.1524) (layer F.Cu) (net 21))
 (segment (start 155.956 107.442) (end 159.512 110.998) (width 0.1524) (layer B.Cu) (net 21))
 (segment (start 147.75 105.15) (end 155.708 105.15) (width 0.1524) (layer F.Cu) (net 22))
 (segment (start 155.708 105.15) (end 155.956 104.902) (width 0.1524) (layer F.Cu) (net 22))
 (segment (start 155.956 104.902) (end 157.048 105.994) (width 0.1524) (layer F.Cu) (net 22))
 (segment (start 157.048 105.994) (end 157.048 109.753) (width 0.1524) (layer F.Cu) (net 22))
 (segment (start 157.048 109.753) (end 156.972 109.83) (width 0.1524) (layer F.Cu) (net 22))
 (segment (start 156.972 109.83) (end 156.972 110.998) (width 0.1524) (layer F.Cu) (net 22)))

